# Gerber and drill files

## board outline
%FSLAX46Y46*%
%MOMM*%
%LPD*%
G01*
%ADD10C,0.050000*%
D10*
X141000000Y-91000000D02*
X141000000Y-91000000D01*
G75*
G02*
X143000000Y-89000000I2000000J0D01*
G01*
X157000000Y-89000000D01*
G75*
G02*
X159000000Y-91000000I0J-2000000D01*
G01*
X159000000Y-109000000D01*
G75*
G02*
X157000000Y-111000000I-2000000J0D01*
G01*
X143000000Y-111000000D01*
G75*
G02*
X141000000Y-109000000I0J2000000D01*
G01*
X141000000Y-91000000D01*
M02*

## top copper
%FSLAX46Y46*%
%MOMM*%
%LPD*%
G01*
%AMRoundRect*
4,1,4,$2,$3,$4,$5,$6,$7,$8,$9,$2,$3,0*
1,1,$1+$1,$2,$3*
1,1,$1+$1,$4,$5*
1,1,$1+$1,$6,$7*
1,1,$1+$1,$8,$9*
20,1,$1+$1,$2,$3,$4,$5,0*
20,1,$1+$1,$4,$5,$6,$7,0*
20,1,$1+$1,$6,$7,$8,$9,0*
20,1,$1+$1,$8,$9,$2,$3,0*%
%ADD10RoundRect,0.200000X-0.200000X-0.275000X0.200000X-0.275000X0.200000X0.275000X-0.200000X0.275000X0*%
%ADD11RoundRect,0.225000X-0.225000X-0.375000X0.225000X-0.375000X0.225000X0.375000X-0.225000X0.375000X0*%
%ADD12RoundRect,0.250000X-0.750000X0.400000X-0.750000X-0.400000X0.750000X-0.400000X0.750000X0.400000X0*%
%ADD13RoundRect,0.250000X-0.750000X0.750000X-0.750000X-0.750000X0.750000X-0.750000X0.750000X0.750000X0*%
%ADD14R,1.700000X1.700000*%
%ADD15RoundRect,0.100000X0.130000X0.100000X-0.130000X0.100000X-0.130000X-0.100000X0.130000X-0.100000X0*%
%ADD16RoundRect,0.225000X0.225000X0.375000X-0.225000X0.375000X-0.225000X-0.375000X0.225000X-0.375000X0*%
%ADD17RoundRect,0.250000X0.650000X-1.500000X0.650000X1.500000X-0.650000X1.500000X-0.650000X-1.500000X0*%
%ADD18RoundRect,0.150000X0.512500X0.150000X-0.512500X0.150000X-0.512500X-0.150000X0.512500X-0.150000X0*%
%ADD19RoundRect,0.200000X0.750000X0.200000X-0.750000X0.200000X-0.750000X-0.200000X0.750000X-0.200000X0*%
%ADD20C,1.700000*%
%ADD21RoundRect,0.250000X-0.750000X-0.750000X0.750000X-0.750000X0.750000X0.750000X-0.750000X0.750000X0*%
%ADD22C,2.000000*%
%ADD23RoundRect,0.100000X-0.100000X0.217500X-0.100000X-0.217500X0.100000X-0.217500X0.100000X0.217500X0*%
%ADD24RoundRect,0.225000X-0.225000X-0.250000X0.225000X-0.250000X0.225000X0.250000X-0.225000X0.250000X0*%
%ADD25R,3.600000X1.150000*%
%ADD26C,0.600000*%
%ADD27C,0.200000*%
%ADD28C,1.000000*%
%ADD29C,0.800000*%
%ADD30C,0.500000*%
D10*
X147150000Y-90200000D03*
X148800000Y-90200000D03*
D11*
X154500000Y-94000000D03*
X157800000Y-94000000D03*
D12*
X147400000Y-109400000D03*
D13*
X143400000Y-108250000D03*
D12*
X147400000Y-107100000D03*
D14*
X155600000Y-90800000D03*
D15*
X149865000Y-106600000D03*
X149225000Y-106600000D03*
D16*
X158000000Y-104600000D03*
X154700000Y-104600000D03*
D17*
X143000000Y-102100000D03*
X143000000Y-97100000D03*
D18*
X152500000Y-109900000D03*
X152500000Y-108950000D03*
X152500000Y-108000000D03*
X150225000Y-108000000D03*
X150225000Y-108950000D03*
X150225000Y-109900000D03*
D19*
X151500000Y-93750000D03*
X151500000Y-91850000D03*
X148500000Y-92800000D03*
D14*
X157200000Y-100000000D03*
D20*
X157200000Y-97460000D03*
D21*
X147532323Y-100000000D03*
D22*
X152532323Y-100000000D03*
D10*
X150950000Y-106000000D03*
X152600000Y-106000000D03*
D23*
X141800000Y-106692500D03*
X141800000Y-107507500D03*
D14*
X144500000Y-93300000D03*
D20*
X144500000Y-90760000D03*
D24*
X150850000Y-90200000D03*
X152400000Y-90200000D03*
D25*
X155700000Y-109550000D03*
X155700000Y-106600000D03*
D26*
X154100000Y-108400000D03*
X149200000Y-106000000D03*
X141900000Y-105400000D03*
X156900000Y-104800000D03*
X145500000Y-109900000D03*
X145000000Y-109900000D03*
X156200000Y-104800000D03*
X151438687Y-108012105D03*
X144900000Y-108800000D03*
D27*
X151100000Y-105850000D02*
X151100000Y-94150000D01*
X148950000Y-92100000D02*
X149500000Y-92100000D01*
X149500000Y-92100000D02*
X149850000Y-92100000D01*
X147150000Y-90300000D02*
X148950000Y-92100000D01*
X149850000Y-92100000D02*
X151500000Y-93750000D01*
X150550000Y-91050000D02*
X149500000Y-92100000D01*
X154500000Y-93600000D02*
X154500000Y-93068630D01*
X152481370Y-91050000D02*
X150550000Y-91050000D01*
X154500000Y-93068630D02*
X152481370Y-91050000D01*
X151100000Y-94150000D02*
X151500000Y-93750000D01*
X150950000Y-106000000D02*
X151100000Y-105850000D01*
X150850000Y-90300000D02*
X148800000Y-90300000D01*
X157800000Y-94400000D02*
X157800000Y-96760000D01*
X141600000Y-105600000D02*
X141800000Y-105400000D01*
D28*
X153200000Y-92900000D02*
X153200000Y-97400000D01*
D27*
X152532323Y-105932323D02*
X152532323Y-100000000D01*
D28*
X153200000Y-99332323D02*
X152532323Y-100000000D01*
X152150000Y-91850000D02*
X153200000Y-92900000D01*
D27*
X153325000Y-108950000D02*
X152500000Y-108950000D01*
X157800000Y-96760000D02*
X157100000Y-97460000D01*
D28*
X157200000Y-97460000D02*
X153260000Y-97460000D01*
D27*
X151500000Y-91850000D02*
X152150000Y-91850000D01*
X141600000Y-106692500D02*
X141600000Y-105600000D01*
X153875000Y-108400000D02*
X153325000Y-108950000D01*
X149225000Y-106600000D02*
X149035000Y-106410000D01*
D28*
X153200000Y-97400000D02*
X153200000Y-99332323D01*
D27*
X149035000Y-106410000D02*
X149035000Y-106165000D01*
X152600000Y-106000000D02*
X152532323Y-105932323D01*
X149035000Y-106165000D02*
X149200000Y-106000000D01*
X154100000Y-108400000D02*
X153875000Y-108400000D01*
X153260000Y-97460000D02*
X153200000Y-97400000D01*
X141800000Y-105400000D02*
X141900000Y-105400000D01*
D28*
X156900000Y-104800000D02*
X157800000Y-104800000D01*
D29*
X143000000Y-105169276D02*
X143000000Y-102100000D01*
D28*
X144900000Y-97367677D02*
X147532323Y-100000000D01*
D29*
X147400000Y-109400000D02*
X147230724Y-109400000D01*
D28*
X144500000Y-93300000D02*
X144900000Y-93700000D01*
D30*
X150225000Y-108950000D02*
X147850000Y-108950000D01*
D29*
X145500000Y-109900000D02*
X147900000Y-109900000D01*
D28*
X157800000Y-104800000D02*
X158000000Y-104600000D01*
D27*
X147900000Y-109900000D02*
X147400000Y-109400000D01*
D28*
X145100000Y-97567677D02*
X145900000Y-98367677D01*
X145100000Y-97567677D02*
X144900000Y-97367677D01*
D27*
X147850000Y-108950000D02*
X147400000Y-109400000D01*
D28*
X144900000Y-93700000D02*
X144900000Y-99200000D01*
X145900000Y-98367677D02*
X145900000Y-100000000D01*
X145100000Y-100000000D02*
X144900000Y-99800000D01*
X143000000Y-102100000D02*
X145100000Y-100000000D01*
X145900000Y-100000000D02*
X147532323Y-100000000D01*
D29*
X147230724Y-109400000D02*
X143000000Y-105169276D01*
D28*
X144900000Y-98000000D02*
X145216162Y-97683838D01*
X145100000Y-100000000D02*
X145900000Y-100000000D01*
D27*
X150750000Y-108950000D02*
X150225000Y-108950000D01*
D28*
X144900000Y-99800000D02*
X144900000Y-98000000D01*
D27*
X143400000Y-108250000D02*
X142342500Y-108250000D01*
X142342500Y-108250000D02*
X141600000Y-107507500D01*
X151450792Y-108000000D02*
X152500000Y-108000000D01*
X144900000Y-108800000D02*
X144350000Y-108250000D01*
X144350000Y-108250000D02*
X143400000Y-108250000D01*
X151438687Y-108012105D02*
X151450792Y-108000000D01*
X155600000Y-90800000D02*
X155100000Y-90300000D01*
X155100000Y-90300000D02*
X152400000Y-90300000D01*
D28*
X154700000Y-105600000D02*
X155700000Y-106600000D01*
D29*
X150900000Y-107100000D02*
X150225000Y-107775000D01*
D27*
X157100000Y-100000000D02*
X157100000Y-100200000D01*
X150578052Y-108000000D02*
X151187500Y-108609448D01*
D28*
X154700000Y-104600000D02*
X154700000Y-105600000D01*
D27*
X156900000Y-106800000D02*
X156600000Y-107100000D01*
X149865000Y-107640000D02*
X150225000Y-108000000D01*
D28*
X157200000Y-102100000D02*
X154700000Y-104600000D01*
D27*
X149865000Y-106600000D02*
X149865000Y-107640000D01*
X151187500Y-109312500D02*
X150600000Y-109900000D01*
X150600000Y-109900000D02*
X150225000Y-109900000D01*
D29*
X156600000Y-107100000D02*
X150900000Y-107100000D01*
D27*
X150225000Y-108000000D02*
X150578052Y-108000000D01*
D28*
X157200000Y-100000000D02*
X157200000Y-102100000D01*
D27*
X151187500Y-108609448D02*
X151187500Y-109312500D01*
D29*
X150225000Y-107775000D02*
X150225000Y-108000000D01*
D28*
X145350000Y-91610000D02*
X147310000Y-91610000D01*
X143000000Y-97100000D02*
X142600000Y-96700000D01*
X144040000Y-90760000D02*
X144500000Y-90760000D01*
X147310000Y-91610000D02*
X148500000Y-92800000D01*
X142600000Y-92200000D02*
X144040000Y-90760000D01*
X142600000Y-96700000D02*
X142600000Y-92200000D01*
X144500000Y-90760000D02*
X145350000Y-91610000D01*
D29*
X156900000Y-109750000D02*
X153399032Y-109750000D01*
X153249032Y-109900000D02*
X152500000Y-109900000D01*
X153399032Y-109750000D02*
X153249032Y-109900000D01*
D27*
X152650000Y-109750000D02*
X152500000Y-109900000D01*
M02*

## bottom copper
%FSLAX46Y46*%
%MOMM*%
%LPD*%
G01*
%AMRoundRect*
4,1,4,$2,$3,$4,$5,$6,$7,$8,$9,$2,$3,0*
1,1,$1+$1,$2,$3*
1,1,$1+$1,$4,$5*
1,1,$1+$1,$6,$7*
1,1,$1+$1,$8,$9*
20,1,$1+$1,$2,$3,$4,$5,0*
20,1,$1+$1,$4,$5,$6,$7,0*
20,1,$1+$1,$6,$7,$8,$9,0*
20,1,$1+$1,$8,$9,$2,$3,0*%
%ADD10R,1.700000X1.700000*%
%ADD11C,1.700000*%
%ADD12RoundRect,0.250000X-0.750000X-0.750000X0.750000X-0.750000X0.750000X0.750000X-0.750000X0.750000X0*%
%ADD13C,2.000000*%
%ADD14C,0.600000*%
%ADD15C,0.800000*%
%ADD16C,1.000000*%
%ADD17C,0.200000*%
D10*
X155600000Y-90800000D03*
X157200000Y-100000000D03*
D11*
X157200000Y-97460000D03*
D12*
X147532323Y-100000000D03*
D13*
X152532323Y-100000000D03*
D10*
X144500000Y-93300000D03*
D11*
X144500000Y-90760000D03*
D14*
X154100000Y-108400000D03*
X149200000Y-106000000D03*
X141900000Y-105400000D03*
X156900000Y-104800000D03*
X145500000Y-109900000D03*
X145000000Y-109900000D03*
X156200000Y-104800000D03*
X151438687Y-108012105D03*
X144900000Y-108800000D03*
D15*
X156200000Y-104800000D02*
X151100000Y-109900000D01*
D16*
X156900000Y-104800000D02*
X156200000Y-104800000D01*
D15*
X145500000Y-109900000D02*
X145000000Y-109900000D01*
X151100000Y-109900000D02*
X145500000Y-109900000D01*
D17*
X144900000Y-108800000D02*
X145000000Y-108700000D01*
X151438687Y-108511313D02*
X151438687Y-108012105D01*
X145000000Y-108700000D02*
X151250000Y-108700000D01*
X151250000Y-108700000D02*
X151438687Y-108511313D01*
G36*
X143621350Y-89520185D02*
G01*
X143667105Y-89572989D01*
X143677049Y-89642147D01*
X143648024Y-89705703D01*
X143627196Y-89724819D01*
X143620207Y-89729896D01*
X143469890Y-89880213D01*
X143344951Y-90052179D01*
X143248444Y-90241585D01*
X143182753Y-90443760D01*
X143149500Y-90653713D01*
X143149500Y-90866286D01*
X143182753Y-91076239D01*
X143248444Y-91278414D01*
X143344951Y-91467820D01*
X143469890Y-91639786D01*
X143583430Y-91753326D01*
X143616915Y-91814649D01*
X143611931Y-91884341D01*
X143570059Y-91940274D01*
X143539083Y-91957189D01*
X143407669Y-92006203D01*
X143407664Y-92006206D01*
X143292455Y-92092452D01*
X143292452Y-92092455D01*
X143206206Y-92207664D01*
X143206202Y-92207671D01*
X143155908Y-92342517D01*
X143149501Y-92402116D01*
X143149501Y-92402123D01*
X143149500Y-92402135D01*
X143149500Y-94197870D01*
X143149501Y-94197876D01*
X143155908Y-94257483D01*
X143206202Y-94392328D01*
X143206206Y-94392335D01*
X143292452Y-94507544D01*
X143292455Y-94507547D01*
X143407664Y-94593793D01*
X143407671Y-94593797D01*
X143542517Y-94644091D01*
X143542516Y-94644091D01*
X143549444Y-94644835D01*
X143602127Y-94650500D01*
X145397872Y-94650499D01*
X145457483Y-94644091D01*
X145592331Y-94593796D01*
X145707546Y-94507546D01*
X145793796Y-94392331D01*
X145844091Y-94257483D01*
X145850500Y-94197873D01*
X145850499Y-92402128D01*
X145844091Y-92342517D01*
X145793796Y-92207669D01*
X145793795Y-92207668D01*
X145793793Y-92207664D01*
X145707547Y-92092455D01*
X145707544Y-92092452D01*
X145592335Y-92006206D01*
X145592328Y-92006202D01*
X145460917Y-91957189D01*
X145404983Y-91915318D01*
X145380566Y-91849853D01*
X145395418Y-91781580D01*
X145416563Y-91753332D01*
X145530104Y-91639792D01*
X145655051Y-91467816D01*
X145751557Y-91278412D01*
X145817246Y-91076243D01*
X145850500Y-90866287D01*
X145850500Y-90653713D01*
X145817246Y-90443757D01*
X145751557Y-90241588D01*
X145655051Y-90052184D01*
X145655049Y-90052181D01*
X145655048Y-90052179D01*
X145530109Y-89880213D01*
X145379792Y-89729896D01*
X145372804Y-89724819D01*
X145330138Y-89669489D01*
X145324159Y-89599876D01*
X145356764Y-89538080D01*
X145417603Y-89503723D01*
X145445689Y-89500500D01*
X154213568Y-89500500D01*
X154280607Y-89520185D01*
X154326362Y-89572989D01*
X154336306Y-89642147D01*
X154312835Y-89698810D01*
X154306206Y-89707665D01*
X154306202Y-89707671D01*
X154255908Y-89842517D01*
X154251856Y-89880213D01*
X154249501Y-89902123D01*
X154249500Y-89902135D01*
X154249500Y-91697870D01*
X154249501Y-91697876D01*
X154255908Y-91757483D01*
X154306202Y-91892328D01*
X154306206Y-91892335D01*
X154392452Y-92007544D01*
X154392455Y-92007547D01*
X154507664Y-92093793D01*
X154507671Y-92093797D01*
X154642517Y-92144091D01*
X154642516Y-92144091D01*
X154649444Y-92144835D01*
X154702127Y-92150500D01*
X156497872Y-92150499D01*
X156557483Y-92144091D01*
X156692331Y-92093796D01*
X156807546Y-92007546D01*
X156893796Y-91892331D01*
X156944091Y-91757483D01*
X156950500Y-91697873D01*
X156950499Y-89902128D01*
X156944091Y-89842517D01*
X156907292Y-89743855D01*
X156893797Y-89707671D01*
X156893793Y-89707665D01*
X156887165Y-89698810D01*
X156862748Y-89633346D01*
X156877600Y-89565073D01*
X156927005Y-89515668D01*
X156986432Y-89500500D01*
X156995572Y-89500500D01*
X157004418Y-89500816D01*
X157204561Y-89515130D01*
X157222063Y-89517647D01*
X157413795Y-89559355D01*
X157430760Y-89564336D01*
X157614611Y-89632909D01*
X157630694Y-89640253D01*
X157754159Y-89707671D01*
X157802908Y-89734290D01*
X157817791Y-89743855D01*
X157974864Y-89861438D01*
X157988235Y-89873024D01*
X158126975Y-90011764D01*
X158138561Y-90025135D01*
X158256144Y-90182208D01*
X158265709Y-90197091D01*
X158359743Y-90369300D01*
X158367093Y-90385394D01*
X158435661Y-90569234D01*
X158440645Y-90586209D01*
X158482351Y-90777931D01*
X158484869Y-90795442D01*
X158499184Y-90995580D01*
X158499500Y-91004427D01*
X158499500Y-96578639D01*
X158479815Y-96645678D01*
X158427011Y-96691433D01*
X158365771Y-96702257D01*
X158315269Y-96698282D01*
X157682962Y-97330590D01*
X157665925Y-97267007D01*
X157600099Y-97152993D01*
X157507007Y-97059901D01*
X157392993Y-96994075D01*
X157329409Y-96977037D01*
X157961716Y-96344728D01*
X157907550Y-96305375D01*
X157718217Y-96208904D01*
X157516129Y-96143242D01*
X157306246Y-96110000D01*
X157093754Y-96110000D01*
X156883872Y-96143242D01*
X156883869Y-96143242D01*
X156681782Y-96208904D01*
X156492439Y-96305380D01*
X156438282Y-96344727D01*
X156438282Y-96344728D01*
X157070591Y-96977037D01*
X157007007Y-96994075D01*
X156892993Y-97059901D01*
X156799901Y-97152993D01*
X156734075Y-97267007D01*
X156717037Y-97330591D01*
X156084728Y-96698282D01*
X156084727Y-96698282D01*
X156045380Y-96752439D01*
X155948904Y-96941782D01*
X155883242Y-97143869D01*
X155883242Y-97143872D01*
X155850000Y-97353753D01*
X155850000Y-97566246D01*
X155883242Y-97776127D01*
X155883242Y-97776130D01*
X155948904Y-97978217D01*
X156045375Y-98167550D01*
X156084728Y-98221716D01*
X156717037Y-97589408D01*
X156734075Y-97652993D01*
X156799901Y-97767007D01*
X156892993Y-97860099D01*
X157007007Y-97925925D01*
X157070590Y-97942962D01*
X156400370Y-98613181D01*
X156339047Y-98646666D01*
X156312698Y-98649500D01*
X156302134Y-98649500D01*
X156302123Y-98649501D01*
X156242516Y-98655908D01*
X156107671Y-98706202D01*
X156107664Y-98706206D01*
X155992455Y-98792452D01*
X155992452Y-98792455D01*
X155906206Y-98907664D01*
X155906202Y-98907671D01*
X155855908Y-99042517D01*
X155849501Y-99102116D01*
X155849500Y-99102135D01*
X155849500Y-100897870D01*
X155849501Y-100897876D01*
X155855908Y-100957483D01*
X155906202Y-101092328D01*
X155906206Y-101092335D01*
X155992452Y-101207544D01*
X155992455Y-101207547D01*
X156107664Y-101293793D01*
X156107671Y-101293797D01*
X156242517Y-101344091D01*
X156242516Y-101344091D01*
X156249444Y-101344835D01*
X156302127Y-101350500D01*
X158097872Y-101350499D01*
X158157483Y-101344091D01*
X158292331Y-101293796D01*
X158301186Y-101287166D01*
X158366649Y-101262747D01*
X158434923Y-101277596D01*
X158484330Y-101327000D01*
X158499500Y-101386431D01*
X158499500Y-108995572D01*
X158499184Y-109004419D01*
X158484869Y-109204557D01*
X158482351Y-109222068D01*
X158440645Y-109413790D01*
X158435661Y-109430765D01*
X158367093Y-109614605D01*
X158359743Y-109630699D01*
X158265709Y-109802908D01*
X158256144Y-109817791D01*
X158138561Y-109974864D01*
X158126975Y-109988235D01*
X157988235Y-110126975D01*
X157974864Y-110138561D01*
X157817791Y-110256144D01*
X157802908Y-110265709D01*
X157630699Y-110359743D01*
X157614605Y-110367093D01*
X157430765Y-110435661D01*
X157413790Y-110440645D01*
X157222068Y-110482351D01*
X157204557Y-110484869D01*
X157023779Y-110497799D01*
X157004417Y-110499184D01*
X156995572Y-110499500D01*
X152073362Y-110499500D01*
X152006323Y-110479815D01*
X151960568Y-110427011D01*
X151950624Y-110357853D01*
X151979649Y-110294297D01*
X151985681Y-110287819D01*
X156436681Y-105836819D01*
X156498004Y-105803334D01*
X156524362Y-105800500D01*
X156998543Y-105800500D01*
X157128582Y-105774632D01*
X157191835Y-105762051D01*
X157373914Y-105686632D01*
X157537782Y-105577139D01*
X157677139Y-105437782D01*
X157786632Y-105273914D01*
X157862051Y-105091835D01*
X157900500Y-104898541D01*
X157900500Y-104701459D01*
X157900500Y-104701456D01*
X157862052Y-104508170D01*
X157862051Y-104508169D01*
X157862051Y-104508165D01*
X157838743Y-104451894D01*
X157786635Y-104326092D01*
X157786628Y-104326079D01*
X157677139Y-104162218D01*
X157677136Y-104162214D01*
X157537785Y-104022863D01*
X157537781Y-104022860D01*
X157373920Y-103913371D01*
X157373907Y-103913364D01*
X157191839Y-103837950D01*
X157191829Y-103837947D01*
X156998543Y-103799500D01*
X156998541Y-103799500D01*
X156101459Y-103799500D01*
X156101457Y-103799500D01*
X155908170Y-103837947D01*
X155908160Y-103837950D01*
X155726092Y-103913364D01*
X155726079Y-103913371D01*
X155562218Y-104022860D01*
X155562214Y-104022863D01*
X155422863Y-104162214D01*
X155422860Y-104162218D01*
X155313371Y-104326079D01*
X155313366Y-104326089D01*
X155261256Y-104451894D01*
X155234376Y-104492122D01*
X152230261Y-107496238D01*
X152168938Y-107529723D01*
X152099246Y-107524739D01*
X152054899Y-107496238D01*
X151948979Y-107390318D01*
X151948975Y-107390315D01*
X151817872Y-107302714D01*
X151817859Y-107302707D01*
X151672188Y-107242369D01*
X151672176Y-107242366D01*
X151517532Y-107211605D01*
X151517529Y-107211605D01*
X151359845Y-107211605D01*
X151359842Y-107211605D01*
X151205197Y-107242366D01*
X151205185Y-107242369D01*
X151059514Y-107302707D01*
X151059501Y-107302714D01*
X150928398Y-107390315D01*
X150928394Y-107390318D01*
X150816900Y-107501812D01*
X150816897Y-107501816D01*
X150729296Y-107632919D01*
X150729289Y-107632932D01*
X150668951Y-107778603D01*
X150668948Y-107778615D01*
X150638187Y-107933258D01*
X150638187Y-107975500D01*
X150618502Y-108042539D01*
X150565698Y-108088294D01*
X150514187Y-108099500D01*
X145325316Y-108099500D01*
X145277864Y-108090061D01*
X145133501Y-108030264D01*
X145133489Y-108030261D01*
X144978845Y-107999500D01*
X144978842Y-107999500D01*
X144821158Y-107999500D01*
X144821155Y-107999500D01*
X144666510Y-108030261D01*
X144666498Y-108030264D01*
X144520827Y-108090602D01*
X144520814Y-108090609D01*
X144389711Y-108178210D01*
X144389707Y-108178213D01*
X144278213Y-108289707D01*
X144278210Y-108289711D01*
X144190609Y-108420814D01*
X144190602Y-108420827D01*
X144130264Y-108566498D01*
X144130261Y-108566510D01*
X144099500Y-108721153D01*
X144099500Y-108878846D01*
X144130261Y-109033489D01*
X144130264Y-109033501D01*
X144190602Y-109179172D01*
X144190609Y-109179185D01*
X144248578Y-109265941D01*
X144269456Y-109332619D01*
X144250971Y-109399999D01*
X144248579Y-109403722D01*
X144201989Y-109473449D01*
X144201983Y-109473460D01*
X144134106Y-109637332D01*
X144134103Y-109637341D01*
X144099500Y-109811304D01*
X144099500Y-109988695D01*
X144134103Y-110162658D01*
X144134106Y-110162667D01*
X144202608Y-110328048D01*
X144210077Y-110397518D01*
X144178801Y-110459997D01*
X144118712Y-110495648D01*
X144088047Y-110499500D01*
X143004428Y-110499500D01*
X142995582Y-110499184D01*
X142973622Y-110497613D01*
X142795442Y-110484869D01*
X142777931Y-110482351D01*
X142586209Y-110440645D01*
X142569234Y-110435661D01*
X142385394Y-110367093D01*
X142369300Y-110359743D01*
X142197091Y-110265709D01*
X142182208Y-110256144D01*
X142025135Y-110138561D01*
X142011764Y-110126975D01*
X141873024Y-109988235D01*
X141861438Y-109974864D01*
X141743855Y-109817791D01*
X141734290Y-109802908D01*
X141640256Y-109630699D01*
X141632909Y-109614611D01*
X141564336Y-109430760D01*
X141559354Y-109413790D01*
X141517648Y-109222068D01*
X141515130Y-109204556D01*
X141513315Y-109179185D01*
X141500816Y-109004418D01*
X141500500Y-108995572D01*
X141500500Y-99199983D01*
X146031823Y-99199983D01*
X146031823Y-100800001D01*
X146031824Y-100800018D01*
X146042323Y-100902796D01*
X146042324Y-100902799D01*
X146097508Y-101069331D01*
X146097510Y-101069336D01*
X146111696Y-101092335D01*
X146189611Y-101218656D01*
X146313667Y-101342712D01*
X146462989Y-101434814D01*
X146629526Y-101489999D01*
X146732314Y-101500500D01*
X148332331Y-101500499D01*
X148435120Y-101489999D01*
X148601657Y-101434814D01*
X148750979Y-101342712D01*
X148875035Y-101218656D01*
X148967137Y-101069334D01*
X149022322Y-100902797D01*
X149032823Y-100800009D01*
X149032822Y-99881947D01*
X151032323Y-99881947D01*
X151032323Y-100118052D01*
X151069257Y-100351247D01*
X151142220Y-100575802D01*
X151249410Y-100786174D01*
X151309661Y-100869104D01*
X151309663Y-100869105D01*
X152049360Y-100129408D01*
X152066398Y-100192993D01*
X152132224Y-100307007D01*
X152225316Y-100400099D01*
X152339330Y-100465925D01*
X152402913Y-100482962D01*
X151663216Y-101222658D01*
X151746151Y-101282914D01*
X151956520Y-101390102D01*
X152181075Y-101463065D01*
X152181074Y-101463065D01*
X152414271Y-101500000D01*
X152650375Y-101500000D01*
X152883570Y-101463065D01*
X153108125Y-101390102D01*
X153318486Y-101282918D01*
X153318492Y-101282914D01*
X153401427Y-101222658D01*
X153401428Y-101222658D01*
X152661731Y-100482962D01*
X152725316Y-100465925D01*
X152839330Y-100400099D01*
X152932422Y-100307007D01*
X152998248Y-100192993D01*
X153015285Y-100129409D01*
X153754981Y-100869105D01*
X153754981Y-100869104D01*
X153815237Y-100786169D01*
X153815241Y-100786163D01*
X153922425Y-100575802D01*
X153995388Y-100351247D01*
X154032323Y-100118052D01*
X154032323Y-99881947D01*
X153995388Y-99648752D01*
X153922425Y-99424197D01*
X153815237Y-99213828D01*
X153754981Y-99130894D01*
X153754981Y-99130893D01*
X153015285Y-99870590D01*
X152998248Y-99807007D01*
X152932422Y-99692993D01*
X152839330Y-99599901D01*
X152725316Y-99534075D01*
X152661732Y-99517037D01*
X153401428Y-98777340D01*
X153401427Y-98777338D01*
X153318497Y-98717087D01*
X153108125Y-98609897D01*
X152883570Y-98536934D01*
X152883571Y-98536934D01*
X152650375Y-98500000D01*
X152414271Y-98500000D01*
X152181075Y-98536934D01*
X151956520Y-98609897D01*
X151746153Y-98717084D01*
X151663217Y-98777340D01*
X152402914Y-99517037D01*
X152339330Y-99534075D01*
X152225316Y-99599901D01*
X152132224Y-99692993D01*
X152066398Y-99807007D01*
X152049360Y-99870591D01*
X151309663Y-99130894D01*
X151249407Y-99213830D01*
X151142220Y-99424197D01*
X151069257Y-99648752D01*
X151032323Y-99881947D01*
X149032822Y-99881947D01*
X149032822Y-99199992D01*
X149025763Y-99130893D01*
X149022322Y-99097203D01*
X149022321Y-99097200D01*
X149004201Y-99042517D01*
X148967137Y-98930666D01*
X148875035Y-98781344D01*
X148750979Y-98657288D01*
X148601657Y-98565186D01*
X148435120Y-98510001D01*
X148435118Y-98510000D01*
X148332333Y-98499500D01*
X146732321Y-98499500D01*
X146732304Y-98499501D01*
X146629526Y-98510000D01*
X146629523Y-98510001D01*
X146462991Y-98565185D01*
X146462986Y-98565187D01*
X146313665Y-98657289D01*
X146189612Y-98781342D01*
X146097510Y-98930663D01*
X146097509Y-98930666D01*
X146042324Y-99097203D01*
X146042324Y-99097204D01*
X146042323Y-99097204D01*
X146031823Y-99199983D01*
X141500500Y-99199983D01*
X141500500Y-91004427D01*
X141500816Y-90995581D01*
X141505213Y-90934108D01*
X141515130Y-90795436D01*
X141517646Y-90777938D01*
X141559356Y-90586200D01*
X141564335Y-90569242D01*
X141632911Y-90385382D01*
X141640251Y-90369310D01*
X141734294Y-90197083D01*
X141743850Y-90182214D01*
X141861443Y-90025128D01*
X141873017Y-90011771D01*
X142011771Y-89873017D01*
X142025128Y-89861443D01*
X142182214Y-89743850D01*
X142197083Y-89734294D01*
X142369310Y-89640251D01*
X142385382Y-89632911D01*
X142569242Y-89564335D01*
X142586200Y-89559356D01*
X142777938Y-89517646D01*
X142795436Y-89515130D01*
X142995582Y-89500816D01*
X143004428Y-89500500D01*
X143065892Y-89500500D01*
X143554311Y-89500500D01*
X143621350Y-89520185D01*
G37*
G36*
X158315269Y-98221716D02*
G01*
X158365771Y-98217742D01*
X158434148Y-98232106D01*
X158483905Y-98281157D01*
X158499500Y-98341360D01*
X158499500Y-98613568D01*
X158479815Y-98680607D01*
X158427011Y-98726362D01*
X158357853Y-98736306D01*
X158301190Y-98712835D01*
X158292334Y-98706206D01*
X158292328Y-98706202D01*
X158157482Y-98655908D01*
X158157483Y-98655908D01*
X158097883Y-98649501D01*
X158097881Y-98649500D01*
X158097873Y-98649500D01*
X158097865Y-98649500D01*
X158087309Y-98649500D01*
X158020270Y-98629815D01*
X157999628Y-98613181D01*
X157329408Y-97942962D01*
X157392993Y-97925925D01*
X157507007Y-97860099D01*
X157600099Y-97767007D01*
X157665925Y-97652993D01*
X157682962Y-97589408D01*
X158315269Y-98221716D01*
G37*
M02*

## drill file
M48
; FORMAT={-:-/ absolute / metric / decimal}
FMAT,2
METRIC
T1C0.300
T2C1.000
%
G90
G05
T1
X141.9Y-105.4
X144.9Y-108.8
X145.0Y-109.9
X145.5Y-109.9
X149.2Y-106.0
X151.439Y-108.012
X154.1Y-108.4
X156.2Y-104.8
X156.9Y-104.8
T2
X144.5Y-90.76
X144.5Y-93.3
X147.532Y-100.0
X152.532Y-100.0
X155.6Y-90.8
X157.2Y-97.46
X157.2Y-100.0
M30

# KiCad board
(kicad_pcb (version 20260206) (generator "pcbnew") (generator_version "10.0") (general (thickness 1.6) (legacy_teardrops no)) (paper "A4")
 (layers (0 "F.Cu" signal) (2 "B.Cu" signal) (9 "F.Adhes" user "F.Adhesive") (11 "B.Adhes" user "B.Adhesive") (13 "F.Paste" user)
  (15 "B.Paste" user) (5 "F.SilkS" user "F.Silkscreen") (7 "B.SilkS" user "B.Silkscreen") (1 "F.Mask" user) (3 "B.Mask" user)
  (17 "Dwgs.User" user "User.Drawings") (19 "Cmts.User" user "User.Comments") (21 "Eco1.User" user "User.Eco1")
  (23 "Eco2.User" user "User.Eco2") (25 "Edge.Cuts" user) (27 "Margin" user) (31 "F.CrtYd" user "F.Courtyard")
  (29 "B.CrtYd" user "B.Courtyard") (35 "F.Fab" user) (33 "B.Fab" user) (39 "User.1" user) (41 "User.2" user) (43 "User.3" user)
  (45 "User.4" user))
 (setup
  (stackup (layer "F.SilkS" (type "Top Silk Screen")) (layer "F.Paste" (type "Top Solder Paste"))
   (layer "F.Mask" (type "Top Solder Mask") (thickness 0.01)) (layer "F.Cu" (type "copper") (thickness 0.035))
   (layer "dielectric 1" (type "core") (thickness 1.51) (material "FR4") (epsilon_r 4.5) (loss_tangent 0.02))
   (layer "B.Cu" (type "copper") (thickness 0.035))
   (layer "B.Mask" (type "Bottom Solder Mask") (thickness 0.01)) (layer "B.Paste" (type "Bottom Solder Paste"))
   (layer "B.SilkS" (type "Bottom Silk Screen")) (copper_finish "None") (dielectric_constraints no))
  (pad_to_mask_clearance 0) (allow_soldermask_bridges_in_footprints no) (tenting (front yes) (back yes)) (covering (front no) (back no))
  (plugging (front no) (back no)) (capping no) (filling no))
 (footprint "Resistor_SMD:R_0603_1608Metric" (layer "F.Cu") (at 147.975 90.2)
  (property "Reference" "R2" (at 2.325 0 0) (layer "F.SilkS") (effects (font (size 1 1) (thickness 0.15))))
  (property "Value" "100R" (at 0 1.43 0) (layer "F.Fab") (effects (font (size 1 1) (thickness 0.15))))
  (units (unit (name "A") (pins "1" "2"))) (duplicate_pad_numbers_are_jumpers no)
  (pad "1" smd roundrect (at -0.825 0) (size 0.8 0.95) (layers "F.Cu" "F.Mask" "F.Paste") (roundrect_rratio 0.25) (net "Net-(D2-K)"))
  (pad "2" smd roundrect (at 0.825 0) (size 0.8 0.95) (layers "F.Cu" "F.Mask" "F.Paste") (roundrect_rratio 0.25) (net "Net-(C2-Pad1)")))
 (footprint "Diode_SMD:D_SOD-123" (layer "F.Cu") (at 156.15 94)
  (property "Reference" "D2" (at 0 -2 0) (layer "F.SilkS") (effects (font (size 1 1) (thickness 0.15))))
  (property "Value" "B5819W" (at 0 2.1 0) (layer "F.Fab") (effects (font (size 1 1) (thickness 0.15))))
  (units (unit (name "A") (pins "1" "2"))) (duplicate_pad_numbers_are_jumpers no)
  (pad "1" smd roundrect (at -1.65 0) (size 0.9 1.2) (layers "F.Cu" "F.Mask" "F.Paste") (roundrect_rratio 0.25) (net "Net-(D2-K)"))
  (pad "2" smd roundrect (at 1.65 0) (size 0.9 1.2) (layers "F.Cu" "F.Mask" "F.Paste") (roundrect_rratio 0.25) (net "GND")))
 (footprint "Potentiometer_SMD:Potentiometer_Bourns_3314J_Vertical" (layer "F.Cu") (at 145.4 108.25 -90)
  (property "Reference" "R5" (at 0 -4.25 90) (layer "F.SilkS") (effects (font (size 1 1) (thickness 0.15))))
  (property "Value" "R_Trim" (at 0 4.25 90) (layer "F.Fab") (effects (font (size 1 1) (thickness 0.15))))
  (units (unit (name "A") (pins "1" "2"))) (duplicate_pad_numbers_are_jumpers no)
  (pad "1" smd roundrect (at 1.15 -2 270) (size 1.3 2) (layers "F.Cu" "F.Mask" "F.Paste") (roundrect_rratio 0.192308) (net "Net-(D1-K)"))
  (pad "2" smd roundrect (at 0 2 270) (size 2 2) (layers "F.Cu" "F.Mask" "F.Paste") (roundrect_rratio 0.125) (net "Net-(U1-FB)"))
  (pad "3" smd roundrect (at -1.15 -2 270) (size 1.3 2) (layers "F.Cu" "F.Mask" "F.Paste") (roundrect_rratio 0.192308)))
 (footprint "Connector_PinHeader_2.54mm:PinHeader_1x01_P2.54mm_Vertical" (layer "F.Cu") (at 155.6 90.8)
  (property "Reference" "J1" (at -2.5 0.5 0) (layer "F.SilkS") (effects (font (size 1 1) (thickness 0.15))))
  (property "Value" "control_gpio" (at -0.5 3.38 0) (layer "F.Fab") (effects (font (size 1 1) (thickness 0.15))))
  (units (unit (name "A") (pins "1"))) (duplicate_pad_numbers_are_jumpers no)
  (pad "1" thru_hole rect (at 0 0) (size 1.7 1.7) (drill 1) (layers "*.Cu" "*.Mask") (remove_unused_layers no) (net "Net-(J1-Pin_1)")))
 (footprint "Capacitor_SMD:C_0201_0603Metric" (layer "F.Cu") (at 149.545 106.6 180)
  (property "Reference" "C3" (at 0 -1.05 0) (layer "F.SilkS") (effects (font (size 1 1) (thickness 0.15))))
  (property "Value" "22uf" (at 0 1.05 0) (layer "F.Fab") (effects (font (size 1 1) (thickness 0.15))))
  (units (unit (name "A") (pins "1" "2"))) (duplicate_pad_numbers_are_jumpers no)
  (pad "" smd roundrect (at -0.345 0 180) (size 0.318 0.36) (layers "F.Paste") (roundrect_rratio 0.25))
  (pad "" smd roundrect (at 0.345 0 180) (size 0.318 0.36) (layers "F.Paste") (roundrect_rratio 0.25))
  (pad "1" smd roundrect (at -0.32 0 180) (size 0.46 0.4) (layers "F.Cu" "F.Mask") (roundrect_rratio 0.25) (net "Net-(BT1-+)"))
  (pad "2" smd roundrect (at 0.32 0 180) (size 0.46 0.4) (layers "F.Cu" "F.Mask") (roundrect_rratio 0.25) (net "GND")))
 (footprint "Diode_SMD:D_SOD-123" (layer "F.Cu") (at 156.35 104.6 180)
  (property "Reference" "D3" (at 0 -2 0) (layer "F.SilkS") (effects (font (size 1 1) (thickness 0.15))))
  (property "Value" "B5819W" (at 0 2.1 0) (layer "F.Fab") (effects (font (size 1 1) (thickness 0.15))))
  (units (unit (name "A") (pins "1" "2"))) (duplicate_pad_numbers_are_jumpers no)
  (pad "1" smd roundrect (at -1.65 0 180) (size 0.9 1.2) (layers "F.Cu" "F.Mask" "F.Paste") (roundrect_rratio 0.25) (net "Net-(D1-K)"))
  (pad "2" smd roundrect (at 1.65 0 180) (size 0.9 1.2) (layers "F.Cu" "F.Mask" "F.Paste") (roundrect_rratio 0.25) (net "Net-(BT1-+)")))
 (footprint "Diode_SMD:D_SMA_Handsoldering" (layer "F.Cu") (at 143 99.6 90)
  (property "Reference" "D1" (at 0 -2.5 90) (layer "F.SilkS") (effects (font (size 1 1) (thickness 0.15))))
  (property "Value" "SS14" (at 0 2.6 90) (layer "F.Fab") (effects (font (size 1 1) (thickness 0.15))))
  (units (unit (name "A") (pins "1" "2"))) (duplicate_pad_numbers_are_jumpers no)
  (pad "1" smd roundrect (at -2.5 0 90) (size 3.5 1.8) (layers "F.Cu" "F.Mask" "F.Paste") (roundrect_rratio 0.1388888889) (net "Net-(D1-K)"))
  (pad "2" smd roundrect (at 2.5 0 90) (size 3.5 1.8) (layers "F.Cu" "F.Mask" "F.Paste") (roundrect_rratio 0.1388888889) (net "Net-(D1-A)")))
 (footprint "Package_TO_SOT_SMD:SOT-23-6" (layer "F.Cu") (at 151.3625 108.95 180)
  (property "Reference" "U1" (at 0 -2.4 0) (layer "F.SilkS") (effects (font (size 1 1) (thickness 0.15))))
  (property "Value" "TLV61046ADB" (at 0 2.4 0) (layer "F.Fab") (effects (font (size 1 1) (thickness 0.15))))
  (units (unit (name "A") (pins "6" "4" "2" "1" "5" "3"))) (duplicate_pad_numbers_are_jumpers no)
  (pad "1" smd roundrect (at -1.1375 -0.95 180) (size 1.325 0.6) (layers "F.Cu" "F.Mask" "F.Paste") (roundrect_rratio 0.25)
   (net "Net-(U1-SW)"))
  (pad "2" smd roundrect (at -1.1375 0 180) (size 1.325 0.6) (layers "F.Cu" "F.Mask" "F.Paste") (roundrect_rratio 0.25) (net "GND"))
  (pad "3" smd roundrect (at -1.1375 0.95 180) (size 1.325 0.6) (layers "F.Cu" "F.Mask" "F.Paste") (roundrect_rratio 0.25)
   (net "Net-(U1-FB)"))
  (pad "4" smd roundrect (at 1.1375 0.95 180) (size 1.325 0.6) (layers "F.Cu" "F.Mask" "F.Paste") (roundrect_rratio 0.25)
   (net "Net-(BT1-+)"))
  (pad "5" smd roundrect (at 1.1375 0 180) (size 1.325 0.6) (layers "F.Cu" "F.Mask" "F.Paste") (roundrect_rratio 0.25) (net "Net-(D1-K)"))
  (pad "6" smd roundrect (at 1.1375 -0.95 180) (size 1.325 0.6) (layers "F.Cu" "F.Mask" "F.Paste") (roundrect_rratio 0.25)
   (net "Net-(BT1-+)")))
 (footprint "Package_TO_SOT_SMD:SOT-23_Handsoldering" (layer "F.Cu") (at 150 92.8 180)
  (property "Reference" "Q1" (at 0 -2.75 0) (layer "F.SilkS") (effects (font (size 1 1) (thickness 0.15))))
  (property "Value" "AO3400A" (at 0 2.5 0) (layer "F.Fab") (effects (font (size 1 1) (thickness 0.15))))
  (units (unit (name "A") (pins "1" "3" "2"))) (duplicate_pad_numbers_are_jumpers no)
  (pad "1" smd roundrect (at -1.5 -0.95 180) (size 1.9 0.8) (layers "F.Cu" "F.Mask" "F.Paste") (roundrect_rratio 0.25) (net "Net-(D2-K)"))
  (pad "2" smd roundrect (at -1.5 0.95 180) (size 1.9 0.8) (layers "F.Cu" "F.Mask" "F.Paste") (roundrect_rratio 0.25) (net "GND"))
  (pad "3" smd roundrect (at 1.5 0 180) (size 1.9 0.8) (layers "F.Cu" "F.Mask" "F.Paste") (roundrect_rratio 0.25) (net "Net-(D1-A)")))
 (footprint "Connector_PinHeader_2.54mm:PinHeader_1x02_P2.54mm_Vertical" (layer "F.Cu") (at 157.2 100 180)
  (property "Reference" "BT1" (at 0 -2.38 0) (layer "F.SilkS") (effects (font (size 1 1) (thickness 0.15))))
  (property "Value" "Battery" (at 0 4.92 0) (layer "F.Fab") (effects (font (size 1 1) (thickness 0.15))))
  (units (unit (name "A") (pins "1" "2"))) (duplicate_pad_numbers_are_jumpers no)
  (pad "1" thru_hole rect (at 0 0 180) (size 1.7 1.7) (drill 1) (layers "*.Cu" "*.Mask") (remove_unused_layers no) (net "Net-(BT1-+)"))
  (pad "2" thru_hole circle (at 0 2.54 180) (size 1.7 1.7) (drill 1) (layers "*.Cu" "*.Mask") (remove_unused_layers no) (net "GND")))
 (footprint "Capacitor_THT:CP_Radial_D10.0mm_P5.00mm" (layer "F.Cu") (at 147.532323 100)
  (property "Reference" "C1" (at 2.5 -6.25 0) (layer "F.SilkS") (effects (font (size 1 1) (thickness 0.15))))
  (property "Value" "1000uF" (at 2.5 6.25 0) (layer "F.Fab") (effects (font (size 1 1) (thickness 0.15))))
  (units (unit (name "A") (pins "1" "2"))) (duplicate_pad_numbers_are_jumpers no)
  (pad "1" thru_hole roundrect (at 0 0) (size 2 2) (drill 1) (layers "*.Cu" "*.Mask") (remove_unused_layers no) (roundrect_rratio 0.125)
   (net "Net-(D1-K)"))
  (pad "2" thru_hole circle (at 5 0) (size 2 2) (drill 1) (layers "*.Cu" "*.Mask") (remove_unused_layers no) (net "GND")))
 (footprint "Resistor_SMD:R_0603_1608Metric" (layer "F.Cu") (at 151.775 106)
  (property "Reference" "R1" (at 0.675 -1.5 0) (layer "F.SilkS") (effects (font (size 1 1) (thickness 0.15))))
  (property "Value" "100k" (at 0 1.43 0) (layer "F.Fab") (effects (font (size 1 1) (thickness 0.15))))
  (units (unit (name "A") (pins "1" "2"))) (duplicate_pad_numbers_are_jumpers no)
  (pad "1" smd roundrect (at -0.825 0) (size 0.8 0.95) (layers "F.Cu" "F.Mask" "F.Paste") (roundrect_rratio 0.25) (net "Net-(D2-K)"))
  (pad "2" smd roundrect (at 0.825 0) (size 0.8 0.95) (layers "F.Cu" "F.Mask" "F.Paste") (roundrect_rratio 0.25) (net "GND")))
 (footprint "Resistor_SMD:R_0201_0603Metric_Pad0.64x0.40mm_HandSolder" (layer "F.Cu") (at 141.8 107.1 -90)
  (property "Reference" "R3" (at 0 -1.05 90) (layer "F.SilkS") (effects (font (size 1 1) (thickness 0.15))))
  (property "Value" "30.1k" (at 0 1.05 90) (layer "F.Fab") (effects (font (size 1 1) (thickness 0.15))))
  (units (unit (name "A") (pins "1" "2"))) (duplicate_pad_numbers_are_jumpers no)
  (pad "" smd roundrect (at -0.4325 0 270) (size 0.458 0.36) (layers "F.Paste") (roundrect_rratio 0.25))
  (pad "" smd roundrect (at 0.4325 0 270) (size 0.458 0.36) (layers "F.Paste") (roundrect_rratio 0.25))
  (pad "1" smd roundrect (at -0.4075 0 270) (size 0.635 0.4) (layers "F.Cu" "F.Mask") (roundrect_rratio 0.25) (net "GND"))
  (pad "2" smd roundrect (at 0.4075 0 270) (size 0.635 0.4) (layers "F.Cu" "F.Mask") (roundrect_rratio 0.25) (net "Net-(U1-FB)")))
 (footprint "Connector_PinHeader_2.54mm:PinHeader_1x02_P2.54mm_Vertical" (layer "F.Cu") (at 144.5 93.3 180)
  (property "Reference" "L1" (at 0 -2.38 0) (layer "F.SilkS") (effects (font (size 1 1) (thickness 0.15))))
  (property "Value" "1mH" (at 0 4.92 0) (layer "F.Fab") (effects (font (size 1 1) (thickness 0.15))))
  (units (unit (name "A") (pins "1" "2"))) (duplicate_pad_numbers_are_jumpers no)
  (pad "1" thru_hole rect (at 0 0 180) (size 1.7 1.7) (drill 1) (layers "*.Cu" "*.Mask") (remove_unused_layers no) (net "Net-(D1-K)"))
  (pad "2" thru_hole circle (at 0 2.54 180) (size 1.7 1.7) (drill 1) (layers "*.Cu" "*.Mask") (remove_unused_layers no) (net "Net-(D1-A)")))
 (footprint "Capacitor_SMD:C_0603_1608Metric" (layer "F.Cu") (at 151.625 90.2)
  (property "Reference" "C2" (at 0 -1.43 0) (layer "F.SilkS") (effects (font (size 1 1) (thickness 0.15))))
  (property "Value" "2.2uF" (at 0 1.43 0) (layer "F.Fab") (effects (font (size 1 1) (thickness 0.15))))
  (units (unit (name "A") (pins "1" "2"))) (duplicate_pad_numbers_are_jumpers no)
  (pad "1" smd roundrect (at -0.775 0) (size 0.9 0.95) (layers "F.Cu" "F.Mask" "F.Paste") (roundrect_rratio 0.25) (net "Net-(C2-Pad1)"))
  (pad "2" smd roundrect (at 0.775 0) (size 0.9 0.95) (layers "F.Cu" "F.Mask" "F.Paste") (roundrect_rratio 0.25) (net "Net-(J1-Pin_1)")))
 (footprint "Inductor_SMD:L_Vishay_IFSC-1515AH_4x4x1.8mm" (layer "F.Cu") (at 155.7 108.075 90)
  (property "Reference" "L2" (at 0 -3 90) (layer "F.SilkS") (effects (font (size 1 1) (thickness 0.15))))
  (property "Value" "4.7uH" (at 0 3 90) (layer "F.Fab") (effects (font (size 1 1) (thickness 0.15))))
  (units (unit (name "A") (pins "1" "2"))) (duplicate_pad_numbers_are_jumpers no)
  (pad "1" smd rect (at -1.475 0 90) (size 1.15 3.6) (layers "F.Cu" "F.Mask" "F.Paste") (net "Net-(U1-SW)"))
  (pad "2" smd rect (at 1.475 0 90) (size 1.15 3.6) (layers "F.Cu" "F.Mask" "F.Paste") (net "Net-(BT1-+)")))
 (gr_rect (start 141 89) (end 159 111) (radius 2) (stroke (width 0.05) (type solid)) (fill no) (layer "Edge.Cuts"))
 (segment (start 151.1 105.85) (end 151.1 94.15) (width 0.2) (layer "F.Cu") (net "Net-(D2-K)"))
 (segment (start 148.95 92.1) (end 149.5 92.1) (width 0.2) (layer "F.Cu") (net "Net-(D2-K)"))
 (segment (start 149.5 92.1) (end 149.85 92.1) (width 0.2) (layer "F.Cu") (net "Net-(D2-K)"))
 (segment (start 147.15 90.3) (end 148.95 92.1) (width 0.2) (layer "F.Cu") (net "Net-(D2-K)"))
 (segment (start 149.85 92.1) (end 151.5 93.75) (width 0.2) (layer "F.Cu") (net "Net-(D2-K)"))
 (segment (start 150.55 91.05) (end 149.5 92.1) (width 0.2) (layer "F.Cu") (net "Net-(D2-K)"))
 (segment (start 154.5 93.6) (end 154.5 93.06863) (width 0.2) (layer "F.Cu") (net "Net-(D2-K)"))
 (segment (start 152.48137 91.05) (end 150.55 91.05) (width 0.2) (layer "F.Cu") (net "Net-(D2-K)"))
 (segment (start 154.5 93.06863) (end 152.48137 91.05) (width 0.2) (layer "F.Cu") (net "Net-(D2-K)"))
 (segment (start 151.1 94.15) (end 151.5 93.75) (width 0.2) (layer "F.Cu") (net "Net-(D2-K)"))
 (segment (start 150.95 106) (end 151.1 105.85) (width 0.2) (layer "F.Cu") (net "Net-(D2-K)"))
 (segment (start 150.85 90.3) (end 148.8 90.3) (width 0.2) (layer "F.Cu") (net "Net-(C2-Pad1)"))
 (segment (start 157.8 94.4) (end 157.8 96.76) (width 0.2) (layer "F.Cu") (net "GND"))
 (segment (start 141.6 105.6) (end 141.8 105.4) (width 0.2) (layer "F.Cu") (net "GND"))
 (segment (start 153.2 92.9) (end 153.2 97.4) (width 1) (layer "F.Cu") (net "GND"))
 (segment (start 152.532323 105.932323) (end 152.532323 100) (width 0.2) (layer "F.Cu") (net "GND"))
 (segment (start 153.2 99.332323) (end 152.532323 100) (width 1) (layer "F.Cu") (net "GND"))
 (segment (start 152.15 91.85) (end 153.2 92.9) (width 1) (layer "F.Cu") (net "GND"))
 (segment (start 153.325 108.95) (end 152.5 108.95) (width 0.2) (layer "F.Cu") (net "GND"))
 (segment (start 157.8 96.76) (end 157.1 97.46) (width 0.2) (layer "F.Cu") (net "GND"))
 (segment (start 157.2 97.46) (end 153.26 97.46) (width 1) (layer "F.Cu") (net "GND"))
 (segment (start 151.5 91.85) (end 152.15 91.85) (width 0.2) (layer "F.Cu") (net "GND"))
 (segment (start 141.6 106.6925) (end 141.6 105.6) (width 0.2) (layer "F.Cu") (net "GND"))
 (segment (start 153.875 108.4) (end 153.325 108.95) (width 0.2) (layer "F.Cu") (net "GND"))
 (segment (start 149.225 106.6) (end 149.035 106.41) (width 0.2) (layer "F.Cu") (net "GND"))
 (segment (start 153.2 97.4) (end 153.2 99.332323) (width 1) (layer "F.Cu") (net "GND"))
 (segment (start 149.035 106.41) (end 149.035 106.165) (width 0.2) (layer "F.Cu") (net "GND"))
 (segment (start 152.6 106) (end 152.532323 105.932323) (width 0.2) (layer "F.Cu") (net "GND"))
 (segment (start 149.035 106.165) (end 149.2 106) (width 0.2) (layer "F.Cu") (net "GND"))
 (segment (start 154.1 108.4) (end 153.875 108.4) (width 0.2) (layer "F.Cu") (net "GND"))
 (segment (start 153.26 97.46) (end 153.2 97.4) (width 0.2) (layer "F.Cu") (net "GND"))
 (segment (start 141.8 105.4) (end 141.9 105.4) (width 0.2) (layer "F.Cu") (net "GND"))
 (via (at 154.1 108.4) (size 0.6) (drill 0.3) (layers "F.Cu" "B.Cu") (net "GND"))
 (via (at 149.2 106) (size 0.6) (drill 0.3) (layers "F.Cu" "B.Cu") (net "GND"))
 (via (at 141.9 105.4) (size 0.6) (drill 0.3) (layers "F.Cu" "B.Cu") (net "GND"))
 (segment (start 156.9 104.8) (end 157.8 104.8) (width 1) (layer "F.Cu") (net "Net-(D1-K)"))
 (segment (start 143 105.169276) (end 143 102.1) (width 0.8) (layer "F.Cu") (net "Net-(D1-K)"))
 (segment (start 144.9 97.367677) (end 147.532323 100) (width 1) (layer "F.Cu") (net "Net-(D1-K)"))
 (segment (start 147.4 109.4) (end 147.230724 109.4) (width 0.8) (layer "F.Cu") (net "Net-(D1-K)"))
 (segment (start 144.5 93.3) (end 144.9 93.7) (width 1) (layer "F.Cu") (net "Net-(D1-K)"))
 (segment (start 150.225 108.95) (end 147.85 108.95) (width 0.5) (layer "F.Cu") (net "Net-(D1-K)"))
 (segment (start 145.5 109.9) (end 147.9 109.9) (width 0.8) (layer "F.Cu") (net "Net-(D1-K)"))
 (segment (start 157.8 104.8) (end 158 104.6) (width 1) (layer "F.Cu") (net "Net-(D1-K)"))
 (segment (start 147.9 109.9) (end 147.4 109.4) (width 0.2) (layer "F.Cu") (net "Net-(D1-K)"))
 (segment (start 145.1 97.567677) (end 145.9 98.367677) (width 1) (layer "F.Cu") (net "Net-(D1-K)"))
 (segment (start 145.1 97.567677) (end 144.9 97.367677) (width 1) (layer "F.Cu") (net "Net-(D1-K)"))
 (segment (start 147.85 108.95) (end 147.4 109.4) (width 0.2) (layer "F.Cu") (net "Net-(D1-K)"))
 (segment (start 144.9 93.7) (end 144.9 99.2) (width 1) (layer "F.Cu") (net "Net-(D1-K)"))
 (segment (start 145.9 98.367677) (end 145.9 100) (width 1) (layer "F.Cu") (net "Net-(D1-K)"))
 (segment (start 145.1 100) (end 144.9 99.8) (width 1) (layer "F.Cu") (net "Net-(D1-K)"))
 (segment (start 143 102.1) (end 145.1 100) (width 1) (layer "F.Cu") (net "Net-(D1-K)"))
 (segment (start 145.9 100) (end 147.532323 100) (width 1) (layer "F.Cu") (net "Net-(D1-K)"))
 (segment (start 147.230724 109.4) (end 143 105.169276) (width 0.8) (layer "F.Cu") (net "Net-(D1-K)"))
 (segment (start 144.9 98) (end 145.216162 97.683838) (width 1) (layer "F.Cu") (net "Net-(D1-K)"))
 (segment (start 145.1 100) (end 145.9 100) (width 1) (layer "F.Cu") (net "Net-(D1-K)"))
 (segment (start 150.75 108.95) (end 150.225 108.95) (width 0.2) (layer "F.Cu") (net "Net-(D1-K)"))
 (segment (start 144.9 99.8) (end 144.9 98) (width 1) (layer "F.Cu") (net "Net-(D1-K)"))
 (via (at 156.9 104.8) (size 0.6) (drill 0.3) (layers "F.Cu" "B.Cu") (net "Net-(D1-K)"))
 (via (at 145.5 109.9) (size 0.6) (drill 0.3) (layers "F.Cu" "B.Cu") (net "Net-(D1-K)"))
 (via (at 145 109.9) (size 0.6) (drill 0.3) (layers "F.Cu" "B.Cu") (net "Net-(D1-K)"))
 (via (at 156.2 104.8) (size 0.6) (drill 0.3) (layers "F.Cu" "B.Cu") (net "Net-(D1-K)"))
 (segment (start 156.2 104.8) (end 151.1 109.9) (width 0.8) (layer "B.Cu") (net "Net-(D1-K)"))
 (segment (start 156.9 104.8) (end 156.2 104.8) (width 1) (layer "B.Cu") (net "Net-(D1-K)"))
 (segment (start 145.5 109.9) (end 145 109.9) (width 0.8) (layer "B.Cu") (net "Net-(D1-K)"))
 (segment (start 151.1 109.9) (end 145.5 109.9) (width 0.8) (layer "B.Cu") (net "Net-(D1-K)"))
 (segment (start 143.4 108.25) (end 142.3425 108.25) (width 0.2) (layer "F.Cu") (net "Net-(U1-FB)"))
 (segment (start 142.3425 108.25) (end 141.6 107.5075) (width 0.2) (layer "F.Cu") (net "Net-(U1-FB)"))
 (segment (start 151.450792 108) (end 152.5 108) (width 0.2) (layer "F.Cu") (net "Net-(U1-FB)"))
 (segment (start 144.9 108.8) (end 144.35 108.25) (width 0.2) (layer "F.Cu") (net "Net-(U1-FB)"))
 (segment (start 144.35 108.25) (end 143.4 108.25) (width 0.2) (layer "F.Cu") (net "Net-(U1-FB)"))
 (segment (start 151.438687 108.012105) (end 151.450792 108) (width 0.2) (layer "F.Cu") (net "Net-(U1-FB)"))
 (via (at 151.438687 108.012105) (size 0.6) (drill 0.3) (layers "F.Cu" "B.Cu") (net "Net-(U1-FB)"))
 (via (at 144.9 108.8) (size 0.6) (drill 0.3) (layers "F.Cu" "B.Cu") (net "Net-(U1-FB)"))
 (segment (start 144.9 108.8) (end 145 108.7) (width 0.2) (layer "B.Cu") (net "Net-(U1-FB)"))
 (segment (start 151.438687 108.511313) (end 151.438687 108.012105) (width 0.2) (layer "B.Cu") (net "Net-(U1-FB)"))
 (segment (start 145 108.7) (end 151.25 108.7) (width 0.2) (layer "B.Cu") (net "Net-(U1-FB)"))
 (segment (start 151.25 108.7) (end 151.438687 108.511313) (width 0.2) (layer "B.Cu") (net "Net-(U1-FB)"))
 (segment (start 155.6 90.8) (end 155.1 90.3) (width 0.2) (layer "F.Cu") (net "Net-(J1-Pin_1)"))
 (segment (start 155.1 90.3) (end 152.4 90.3) (width 0.2) (layer "F.Cu") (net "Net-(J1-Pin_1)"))
 (segment (start 154.7 105.6) (end 155.7 106.6) (width 1) (layer "F.Cu") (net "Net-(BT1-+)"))
 (segment (start 150.9 107.1) (end 150.225 107.775) (width 0.8) (layer "F.Cu") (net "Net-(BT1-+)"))
 (segment (start 157.1 100) (end 157.1 100.2) (width 0.2) (layer "F.Cu") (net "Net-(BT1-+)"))
 (segment (start 150.578052 108) (end 151.1875 108.609448) (width 0.2) (layer "F.Cu") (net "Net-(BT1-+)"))
 (segment (start 154.7 104.6) (end 154.7 105.6) (width 1) (layer "F.Cu") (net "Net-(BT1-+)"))
 (segment (start 156.9 106.8) (end 156.6 107.1) (width 0.2) (layer "F.Cu") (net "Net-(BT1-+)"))
 (segment (start 149.865 107.64) (end 150.225 108) (width 0.2) (layer "F.Cu") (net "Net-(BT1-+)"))
 (segment (start 157.2 102.1) (end 154.7 104.6) (width 1) (layer "F.Cu") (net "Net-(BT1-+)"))
 (segment (start 149.865 106.6) (end 149.865 107.64) (width 0.2) (layer "F.Cu") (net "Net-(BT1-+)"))
 (segment (start 151.1875 109.3125) (end 150.6 109.9) (width 0.2) (layer "F.Cu") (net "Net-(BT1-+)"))
 (segment (start 150.6 109.9) (end 150.225 109.9) (width 0.2) (layer "F.Cu") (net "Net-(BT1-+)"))
 (segment (start 156.6 107.1) (end 150.9 107.1) (width 0.8) (layer "F.Cu") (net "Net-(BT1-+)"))
 (segment (start 150.225 108) (end 150.578052 108) (width 0.2) (layer "F.Cu") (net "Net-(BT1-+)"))
 (segment (start 157.2 100) (end 157.2 102.1) (width 1) (layer "F.Cu") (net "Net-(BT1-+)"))
 (segment (start 151.1875 108.609448) (end 151.1875 109.3125) (width 0.2) (layer "F.Cu") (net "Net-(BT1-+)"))
 (segment (start 150.225 107.775) (end 150.225 108) (width 0.8) (layer "F.Cu") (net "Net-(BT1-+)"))
 (segment (start 145.35 91.61) (end 147.31 91.61) (width 1) (layer "F.Cu") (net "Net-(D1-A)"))
 (segment (start 143 97.1) (end 142.6 96.7) (width 1) (layer "F.Cu") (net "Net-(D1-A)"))
 (segment (start 144.04 90.76) (end 144.5 90.76) (width 1) (layer "F.Cu") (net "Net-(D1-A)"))
 (segment (start 147.31 91.61) (end 148.5 92.8) (width 1) (layer "F.Cu") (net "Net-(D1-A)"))
 (segment (start 142.6 92.2) (end 144.04 90.76) (width 1) (layer "F.Cu") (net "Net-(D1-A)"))
 (segment (start 142.6 96.7) (end 142.6 92.2) (width 1) (layer "F.Cu") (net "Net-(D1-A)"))
 (segment (start 144.5 90.76) (end 145.35 91.61) (width 1) (layer "F.Cu") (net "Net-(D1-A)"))
 (segment (start 156.9 109.75) (end 153.399032 109.75) (width 0.8) (layer "F.Cu") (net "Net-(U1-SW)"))
 (segment (start 153.249032 109.9) (end 152.5 109.9) (width 0.8) (layer "F.Cu") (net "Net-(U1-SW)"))
 (segment (start 153.399032 109.75) (end 153.249032 109.9) (width 0.8) (layer "F.Cu") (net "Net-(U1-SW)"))
 (segment (start 152.65 109.75) (end 152.5 109.9) (width 0.2) (layer "F.Cu") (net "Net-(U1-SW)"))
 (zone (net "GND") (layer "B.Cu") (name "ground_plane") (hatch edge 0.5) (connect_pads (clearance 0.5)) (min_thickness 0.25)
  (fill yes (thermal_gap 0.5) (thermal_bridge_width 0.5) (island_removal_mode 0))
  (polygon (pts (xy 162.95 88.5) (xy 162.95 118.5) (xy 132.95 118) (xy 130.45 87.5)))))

